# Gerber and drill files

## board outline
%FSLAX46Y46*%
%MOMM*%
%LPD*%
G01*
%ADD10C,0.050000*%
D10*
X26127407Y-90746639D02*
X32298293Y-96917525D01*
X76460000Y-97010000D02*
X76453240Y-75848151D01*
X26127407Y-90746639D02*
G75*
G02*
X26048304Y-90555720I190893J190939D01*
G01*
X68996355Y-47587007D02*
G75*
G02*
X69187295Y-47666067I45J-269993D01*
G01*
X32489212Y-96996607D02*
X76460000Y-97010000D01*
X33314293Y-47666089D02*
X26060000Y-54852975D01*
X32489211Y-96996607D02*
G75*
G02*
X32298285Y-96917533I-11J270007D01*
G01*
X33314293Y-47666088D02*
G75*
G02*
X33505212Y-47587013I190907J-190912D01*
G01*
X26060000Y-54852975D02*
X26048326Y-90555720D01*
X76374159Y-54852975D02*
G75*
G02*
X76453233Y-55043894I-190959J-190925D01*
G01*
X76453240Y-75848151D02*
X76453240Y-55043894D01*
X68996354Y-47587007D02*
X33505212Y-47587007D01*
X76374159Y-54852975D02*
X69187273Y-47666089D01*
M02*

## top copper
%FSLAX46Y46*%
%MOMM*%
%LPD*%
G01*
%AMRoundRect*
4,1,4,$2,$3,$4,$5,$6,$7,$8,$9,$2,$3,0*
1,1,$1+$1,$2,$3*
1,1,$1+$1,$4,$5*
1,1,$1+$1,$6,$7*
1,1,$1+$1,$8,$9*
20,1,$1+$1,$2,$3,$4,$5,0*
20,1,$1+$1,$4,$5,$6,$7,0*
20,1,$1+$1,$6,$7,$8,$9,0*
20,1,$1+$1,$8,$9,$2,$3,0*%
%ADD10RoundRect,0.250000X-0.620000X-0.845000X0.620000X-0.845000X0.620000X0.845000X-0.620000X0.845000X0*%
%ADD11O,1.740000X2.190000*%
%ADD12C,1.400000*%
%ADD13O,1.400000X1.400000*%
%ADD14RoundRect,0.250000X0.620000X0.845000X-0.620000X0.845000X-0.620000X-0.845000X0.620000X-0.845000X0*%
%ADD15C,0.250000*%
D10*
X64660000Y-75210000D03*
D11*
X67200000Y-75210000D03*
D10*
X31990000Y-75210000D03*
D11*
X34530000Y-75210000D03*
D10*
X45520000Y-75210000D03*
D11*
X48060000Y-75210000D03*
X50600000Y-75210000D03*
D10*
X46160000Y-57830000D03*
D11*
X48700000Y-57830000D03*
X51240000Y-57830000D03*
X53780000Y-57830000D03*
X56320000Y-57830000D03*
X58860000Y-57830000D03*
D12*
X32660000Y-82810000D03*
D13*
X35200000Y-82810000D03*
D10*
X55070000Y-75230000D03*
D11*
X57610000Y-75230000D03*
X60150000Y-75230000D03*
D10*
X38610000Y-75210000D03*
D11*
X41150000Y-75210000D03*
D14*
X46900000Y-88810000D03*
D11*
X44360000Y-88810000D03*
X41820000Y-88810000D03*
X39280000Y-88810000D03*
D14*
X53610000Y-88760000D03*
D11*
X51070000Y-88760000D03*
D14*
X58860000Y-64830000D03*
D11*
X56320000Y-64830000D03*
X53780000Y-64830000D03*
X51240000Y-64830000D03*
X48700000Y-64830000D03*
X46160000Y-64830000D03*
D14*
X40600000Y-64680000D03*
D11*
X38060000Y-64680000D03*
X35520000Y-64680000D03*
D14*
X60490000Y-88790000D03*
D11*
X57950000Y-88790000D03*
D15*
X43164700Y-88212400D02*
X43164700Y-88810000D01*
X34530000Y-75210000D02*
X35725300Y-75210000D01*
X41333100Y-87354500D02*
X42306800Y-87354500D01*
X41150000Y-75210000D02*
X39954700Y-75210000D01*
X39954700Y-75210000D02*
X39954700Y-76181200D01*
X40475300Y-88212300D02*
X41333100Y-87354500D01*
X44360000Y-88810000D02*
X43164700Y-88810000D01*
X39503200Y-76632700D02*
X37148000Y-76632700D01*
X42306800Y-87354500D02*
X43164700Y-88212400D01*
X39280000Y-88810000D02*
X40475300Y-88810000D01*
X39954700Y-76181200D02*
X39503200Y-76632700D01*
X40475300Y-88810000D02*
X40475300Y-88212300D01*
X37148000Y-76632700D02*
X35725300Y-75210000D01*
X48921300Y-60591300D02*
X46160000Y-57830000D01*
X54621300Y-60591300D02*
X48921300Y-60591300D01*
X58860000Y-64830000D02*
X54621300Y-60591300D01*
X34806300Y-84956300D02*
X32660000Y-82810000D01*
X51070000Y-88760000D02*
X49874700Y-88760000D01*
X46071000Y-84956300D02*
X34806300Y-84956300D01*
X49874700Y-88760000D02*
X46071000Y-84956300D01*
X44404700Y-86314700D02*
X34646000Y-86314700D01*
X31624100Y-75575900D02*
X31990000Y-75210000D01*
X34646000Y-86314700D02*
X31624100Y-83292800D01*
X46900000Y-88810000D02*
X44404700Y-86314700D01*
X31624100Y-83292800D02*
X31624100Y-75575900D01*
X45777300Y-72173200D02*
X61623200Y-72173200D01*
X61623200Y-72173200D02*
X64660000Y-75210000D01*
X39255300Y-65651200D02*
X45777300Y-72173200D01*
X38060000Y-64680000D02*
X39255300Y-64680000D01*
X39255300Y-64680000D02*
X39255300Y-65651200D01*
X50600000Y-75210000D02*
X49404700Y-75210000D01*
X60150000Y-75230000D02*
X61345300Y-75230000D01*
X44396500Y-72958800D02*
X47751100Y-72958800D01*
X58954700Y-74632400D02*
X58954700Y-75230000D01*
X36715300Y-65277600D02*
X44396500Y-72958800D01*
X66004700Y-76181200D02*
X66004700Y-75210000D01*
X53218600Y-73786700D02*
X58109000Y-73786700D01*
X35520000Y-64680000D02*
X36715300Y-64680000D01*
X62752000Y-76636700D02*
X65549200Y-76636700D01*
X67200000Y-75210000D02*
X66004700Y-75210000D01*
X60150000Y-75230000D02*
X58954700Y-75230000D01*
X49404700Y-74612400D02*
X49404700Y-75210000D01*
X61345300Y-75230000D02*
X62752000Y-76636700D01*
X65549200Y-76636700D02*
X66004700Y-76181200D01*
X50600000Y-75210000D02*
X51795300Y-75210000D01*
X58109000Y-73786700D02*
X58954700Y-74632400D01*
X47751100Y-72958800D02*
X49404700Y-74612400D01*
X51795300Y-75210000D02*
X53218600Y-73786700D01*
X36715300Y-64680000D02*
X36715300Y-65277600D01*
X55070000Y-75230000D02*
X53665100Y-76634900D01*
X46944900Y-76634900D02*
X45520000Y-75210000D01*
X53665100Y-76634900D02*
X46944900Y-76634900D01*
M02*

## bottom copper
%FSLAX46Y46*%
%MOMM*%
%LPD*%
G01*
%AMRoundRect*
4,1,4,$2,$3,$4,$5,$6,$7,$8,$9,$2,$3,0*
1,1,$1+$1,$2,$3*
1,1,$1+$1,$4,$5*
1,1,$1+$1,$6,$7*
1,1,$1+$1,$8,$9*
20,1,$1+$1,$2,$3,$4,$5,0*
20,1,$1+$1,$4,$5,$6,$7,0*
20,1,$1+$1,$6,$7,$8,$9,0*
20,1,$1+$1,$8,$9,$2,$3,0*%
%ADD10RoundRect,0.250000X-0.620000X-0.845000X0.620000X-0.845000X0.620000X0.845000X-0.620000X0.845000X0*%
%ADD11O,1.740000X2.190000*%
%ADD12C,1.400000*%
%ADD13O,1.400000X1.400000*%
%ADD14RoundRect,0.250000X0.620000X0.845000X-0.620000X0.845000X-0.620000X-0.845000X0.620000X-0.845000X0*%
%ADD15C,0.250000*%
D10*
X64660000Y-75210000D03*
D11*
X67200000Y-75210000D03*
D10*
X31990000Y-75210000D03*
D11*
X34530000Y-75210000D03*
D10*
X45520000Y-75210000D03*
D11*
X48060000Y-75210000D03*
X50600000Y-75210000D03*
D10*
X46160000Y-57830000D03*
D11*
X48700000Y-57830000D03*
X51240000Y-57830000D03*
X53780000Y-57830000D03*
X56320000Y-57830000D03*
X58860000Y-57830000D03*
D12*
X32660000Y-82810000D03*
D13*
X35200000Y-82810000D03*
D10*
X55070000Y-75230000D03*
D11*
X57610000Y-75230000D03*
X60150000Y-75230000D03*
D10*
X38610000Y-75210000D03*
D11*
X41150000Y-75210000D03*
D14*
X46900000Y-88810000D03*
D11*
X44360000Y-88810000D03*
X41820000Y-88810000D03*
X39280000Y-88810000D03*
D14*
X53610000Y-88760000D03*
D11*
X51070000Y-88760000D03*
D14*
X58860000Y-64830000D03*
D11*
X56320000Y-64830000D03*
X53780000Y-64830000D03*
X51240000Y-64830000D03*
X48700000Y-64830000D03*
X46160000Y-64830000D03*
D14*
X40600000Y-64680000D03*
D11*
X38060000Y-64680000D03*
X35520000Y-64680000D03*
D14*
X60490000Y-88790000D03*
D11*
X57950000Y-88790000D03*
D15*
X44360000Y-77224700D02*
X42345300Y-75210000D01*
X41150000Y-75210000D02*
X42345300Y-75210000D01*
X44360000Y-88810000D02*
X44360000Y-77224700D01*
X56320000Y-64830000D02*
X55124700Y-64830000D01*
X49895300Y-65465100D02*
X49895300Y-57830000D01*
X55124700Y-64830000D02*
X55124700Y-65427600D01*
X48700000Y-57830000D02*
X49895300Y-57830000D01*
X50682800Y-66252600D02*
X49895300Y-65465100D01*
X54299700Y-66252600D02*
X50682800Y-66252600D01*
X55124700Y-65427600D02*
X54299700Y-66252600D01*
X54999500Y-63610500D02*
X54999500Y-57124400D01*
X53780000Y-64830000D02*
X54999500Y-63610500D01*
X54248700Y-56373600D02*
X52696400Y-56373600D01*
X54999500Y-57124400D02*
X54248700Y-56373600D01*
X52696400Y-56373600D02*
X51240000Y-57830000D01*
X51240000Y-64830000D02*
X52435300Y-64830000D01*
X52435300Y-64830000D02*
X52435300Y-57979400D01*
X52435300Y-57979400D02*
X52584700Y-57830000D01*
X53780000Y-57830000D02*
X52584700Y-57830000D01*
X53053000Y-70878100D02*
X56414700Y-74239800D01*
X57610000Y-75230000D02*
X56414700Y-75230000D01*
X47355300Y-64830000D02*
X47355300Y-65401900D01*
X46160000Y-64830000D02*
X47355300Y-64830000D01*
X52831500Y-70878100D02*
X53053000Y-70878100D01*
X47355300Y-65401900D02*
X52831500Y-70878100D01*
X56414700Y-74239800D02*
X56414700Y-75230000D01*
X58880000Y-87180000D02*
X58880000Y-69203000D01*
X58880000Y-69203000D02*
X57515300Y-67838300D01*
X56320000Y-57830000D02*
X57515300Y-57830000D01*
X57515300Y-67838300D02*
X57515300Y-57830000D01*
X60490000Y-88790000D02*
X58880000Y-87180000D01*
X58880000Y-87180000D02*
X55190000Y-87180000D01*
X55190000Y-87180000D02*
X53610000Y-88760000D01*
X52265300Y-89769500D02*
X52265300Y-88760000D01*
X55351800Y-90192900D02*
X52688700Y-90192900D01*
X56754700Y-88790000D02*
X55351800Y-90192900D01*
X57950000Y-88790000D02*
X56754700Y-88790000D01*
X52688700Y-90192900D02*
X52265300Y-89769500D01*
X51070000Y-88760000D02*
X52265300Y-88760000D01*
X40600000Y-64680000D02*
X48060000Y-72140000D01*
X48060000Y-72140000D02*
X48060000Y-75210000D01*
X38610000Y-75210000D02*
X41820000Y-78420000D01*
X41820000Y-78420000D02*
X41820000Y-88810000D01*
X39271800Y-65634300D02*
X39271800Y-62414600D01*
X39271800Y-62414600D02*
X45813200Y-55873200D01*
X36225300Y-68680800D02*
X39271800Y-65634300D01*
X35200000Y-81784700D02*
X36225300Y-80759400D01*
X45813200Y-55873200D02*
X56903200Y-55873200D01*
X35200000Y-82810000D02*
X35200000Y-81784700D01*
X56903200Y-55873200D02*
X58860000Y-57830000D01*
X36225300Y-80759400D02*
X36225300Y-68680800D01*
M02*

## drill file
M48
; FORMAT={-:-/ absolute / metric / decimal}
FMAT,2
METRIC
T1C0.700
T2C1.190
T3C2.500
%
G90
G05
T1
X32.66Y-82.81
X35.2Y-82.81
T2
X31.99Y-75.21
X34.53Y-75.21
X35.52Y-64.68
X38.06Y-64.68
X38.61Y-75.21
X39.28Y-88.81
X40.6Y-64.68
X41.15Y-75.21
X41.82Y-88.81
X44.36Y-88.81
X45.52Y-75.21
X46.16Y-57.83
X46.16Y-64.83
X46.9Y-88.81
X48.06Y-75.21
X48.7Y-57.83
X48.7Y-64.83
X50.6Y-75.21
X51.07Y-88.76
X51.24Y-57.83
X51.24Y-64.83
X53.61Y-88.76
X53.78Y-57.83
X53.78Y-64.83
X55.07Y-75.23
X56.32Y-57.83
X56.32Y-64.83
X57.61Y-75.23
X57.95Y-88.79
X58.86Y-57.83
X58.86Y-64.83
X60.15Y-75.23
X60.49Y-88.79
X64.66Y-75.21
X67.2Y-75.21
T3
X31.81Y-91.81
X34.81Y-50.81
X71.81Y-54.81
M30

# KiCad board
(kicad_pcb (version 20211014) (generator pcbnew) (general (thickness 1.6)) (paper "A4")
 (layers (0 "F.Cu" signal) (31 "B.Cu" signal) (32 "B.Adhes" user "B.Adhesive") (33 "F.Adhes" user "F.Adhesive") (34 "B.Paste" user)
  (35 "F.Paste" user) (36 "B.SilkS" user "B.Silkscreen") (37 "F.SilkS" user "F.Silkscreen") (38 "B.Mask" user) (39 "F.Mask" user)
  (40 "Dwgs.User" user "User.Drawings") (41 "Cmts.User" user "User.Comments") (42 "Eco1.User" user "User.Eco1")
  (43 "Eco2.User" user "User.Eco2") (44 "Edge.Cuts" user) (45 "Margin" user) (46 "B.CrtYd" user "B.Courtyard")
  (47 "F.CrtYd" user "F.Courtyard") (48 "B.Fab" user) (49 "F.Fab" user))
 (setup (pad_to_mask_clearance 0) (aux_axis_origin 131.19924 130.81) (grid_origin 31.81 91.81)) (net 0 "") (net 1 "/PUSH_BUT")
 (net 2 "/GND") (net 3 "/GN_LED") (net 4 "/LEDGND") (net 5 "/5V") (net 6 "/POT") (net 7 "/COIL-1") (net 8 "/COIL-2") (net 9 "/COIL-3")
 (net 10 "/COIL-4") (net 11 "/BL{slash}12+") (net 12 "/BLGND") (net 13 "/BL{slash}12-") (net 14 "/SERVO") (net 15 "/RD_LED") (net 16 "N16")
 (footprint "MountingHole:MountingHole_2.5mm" (layer "F.Cu") (at 34.81 50.81)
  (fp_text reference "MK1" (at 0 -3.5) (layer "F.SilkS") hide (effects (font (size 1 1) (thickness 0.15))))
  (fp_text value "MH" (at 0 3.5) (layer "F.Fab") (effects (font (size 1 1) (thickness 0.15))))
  (pad "" np_thru_hole circle locked (at 0 0) (size 2.5 2.5) (drill 2.5) (layers *.Cu *.Mask)))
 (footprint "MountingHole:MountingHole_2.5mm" (layer "F.Cu") (at 31.81 91.81)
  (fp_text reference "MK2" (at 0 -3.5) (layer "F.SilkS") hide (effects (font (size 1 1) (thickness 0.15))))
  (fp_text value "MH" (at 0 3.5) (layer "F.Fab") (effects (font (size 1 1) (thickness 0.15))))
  (pad "" np_thru_hole circle locked (at 0 0) (size 2.5 2.5) (drill 2.5) (layers *.Cu *.Mask)))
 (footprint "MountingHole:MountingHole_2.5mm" (layer "F.Cu") (at 71.81 54.81)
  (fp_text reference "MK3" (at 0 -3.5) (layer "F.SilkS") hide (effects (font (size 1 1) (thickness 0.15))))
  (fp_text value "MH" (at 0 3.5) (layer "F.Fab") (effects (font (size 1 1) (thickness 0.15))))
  (pad "" np_thru_hole circle locked (at 0 0) (size 2.5 2.5) (drill 2.5) (layers *.Cu *.Mask)))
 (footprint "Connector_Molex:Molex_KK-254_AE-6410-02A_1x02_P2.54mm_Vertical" (layer "F.Cu") (at 64.66 75.21)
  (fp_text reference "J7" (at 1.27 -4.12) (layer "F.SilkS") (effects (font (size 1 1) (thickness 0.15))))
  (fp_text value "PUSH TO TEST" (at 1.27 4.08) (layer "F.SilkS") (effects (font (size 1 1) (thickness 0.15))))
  (pad "1" thru_hole roundrect (at 0 0) (size 1.74 2.19) (drill 1.19) (layers *.Cu *.Mask) (roundrect_rratio 0.1436781609)
   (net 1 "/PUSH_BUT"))
  (pad "2" thru_hole oval (at 2.54 0) (size 1.74 2.19) (drill 1.19) (layers *.Cu *.Mask) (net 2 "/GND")))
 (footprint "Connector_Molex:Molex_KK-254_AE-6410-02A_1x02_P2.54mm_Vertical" (layer "F.Cu") (at 31.99 75.21)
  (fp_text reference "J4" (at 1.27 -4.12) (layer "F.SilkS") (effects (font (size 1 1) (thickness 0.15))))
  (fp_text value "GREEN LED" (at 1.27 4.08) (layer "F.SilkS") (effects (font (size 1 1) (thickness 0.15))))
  (pad "1" thru_hole roundrect (at 0 0) (size 1.74 2.19) (drill 1.19) (layers *.Cu *.Mask) (roundrect_rratio 0.1436781609) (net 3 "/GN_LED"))
  (pad "2" thru_hole oval (at 2.54 0) (size 1.74 2.19) (drill 1.19) (layers *.Cu *.Mask) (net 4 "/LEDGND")))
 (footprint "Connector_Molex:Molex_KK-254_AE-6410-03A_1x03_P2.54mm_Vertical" (layer "F.Cu") (at 45.52 75.21)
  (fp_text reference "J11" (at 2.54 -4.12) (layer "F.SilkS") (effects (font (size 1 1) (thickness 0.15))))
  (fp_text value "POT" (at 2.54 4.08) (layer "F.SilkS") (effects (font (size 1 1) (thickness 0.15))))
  (pad "1" thru_hole roundrect (at 0 0) (size 1.74 2.19) (drill 1.19) (layers *.Cu *.Mask) (roundrect_rratio 0.1436781609) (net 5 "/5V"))
  (pad "2" thru_hole oval (at 2.54 0) (size 1.74 2.19) (drill 1.19) (layers *.Cu *.Mask) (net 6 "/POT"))
  (pad "3" thru_hole oval (at 5.08 0) (size 1.74 2.19) (drill 1.19) (layers *.Cu *.Mask) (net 2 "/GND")))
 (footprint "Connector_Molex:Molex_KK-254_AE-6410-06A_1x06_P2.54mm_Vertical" (layer "F.Cu") (at 46.16 57.83)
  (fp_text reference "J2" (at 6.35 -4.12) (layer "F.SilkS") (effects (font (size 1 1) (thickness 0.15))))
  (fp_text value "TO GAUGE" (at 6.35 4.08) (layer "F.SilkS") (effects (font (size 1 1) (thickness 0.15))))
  (pad "1" thru_hole roundrect (at 0 0) (size 1.74 2.19) (drill 1.19) (layers *.Cu *.Mask) (roundrect_rratio 0.1436781609) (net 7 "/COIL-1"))
  (pad "2" thru_hole oval (at 2.54 0) (size 1.74 2.19) (drill 1.19) (layers *.Cu *.Mask) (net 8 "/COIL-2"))
  (pad "3" thru_hole oval (at 5.08 0) (size 1.74 2.19) (drill 1.19) (layers *.Cu *.Mask) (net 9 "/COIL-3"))
  (pad "4" thru_hole oval (at 7.62 0) (size 1.74 2.19) (drill 1.19) (layers *.Cu *.Mask) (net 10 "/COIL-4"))
  (pad "5" thru_hole oval (at 10.16 0) (size 1.74 2.19) (drill 1.19) (layers *.Cu *.Mask) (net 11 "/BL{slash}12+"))
  (pad "6" thru_hole oval (at 12.7 0) (size 1.74 2.19) (drill 1.19) (layers *.Cu *.Mask) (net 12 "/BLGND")))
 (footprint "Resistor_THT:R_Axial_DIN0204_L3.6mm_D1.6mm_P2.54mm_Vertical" (layer "F.Cu") (at 32.66 82.81)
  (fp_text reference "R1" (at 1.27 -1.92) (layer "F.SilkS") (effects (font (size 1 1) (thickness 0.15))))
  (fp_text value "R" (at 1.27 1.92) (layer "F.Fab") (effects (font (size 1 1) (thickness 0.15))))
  (pad "1" thru_hole circle (at 0 0) (size 1.4 1.4) (drill 0.7) (layers *.Cu *.Mask) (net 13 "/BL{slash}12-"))
  (pad "2" thru_hole oval (at 2.54 0) (size 1.4 1.4) (drill 0.7) (layers *.Cu *.Mask) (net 12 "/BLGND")))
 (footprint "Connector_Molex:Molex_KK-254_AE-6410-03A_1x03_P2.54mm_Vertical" (layer "F.Cu") (at 55.07 75.23)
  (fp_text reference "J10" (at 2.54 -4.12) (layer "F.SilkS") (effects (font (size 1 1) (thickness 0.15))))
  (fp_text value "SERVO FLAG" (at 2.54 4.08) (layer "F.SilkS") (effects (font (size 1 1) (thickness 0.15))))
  (pad "1" thru_hole roundrect (at 0 0) (size 1.74 2.19) (drill 1.19) (layers *.Cu *.Mask) (roundrect_rratio 0.1436781609) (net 5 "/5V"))
  (pad "2" thru_hole oval (at 2.54 0) (size 1.74 2.19) (drill 1.19) (layers *.Cu *.Mask) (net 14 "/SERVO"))
  (pad "3" thru_hole oval (at 5.08 0) (size 1.74 2.19) (drill 1.19) (layers *.Cu *.Mask) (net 2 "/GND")))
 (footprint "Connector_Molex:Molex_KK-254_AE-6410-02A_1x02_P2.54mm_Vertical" (layer "F.Cu") (at 38.61 75.21)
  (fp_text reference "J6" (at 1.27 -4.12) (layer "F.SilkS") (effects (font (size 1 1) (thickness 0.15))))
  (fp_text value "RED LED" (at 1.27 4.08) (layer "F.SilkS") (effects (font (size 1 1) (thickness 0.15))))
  (pad "1" thru_hole roundrect (at 0 0) (size 1.74 2.19) (drill 1.19) (layers *.Cu *.Mask) (roundrect_rratio 0.1436781609)
   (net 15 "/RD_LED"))
  (pad "2" thru_hole oval (at 2.54 0) (size 1.74 2.19) (drill 1.19) (layers *.Cu *.Mask) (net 4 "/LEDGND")))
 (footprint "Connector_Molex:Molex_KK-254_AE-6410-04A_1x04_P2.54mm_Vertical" (layer "B.Cu") (at 46.9 88.81 180)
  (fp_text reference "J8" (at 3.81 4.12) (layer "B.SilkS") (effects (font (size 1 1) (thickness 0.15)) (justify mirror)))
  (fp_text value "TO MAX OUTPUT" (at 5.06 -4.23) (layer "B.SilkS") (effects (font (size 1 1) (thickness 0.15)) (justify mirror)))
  (pad "1" thru_hole roundrect (at 0 0 180) (size 1.74 2.19) (drill 1.19) (layers *.Cu *.Mask) (roundrect_rratio 0.1436781609)
   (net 3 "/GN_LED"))
  (pad "2" thru_hole oval (at 2.54 0 180) (size 1.74 2.19) (drill 1.19) (layers *.Cu *.Mask) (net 4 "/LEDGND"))
  (pad "3" thru_hole oval (at 5.08 0 180) (size 1.74 2.19) (drill 1.19) (layers *.Cu *.Mask) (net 15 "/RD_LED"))
  (pad "4" thru_hole oval (at 7.62 0 180) (size 1.74 2.19) (drill 1.19) (layers *.Cu *.Mask) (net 4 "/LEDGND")))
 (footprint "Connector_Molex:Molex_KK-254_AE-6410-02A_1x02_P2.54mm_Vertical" (layer "B.Cu") (at 53.61 88.76 180)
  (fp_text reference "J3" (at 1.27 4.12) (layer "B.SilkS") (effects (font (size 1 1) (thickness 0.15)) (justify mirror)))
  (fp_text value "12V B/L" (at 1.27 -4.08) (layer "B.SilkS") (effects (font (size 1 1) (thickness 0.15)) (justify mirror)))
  (pad "1" thru_hole roundrect (at 0 0 180) (size 1.74 2.19) (drill 1.19) (layers *.Cu *.Mask) (roundrect_rratio 0.1436781609)
   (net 11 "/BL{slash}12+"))
  (pad "2" thru_hole oval (at 2.54 0 180) (size 1.74 2.19) (drill 1.19) (layers *.Cu *.Mask) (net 13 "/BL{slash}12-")))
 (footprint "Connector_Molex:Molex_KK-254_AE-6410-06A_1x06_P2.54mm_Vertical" (layer "B.Cu") (at 58.86 64.83 180)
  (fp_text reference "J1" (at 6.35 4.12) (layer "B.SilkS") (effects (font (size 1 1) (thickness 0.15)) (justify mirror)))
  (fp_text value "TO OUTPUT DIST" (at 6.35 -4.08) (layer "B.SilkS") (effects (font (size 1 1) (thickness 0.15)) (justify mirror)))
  (pad "1" thru_hole roundrect (at 0 0 180) (size 1.74 2.19) (drill 1.19) (layers *.Cu *.Mask) (roundrect_rratio 0.1436781609)
   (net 7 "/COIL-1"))
  (pad "2" thru_hole oval (at 2.54 0 180) (size 1.74 2.19) (drill 1.19) (layers *.Cu *.Mask) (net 8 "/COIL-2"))
  (pad "3" thru_hole oval (at 5.08 0 180) (size 1.74 2.19) (drill 1.19) (layers *.Cu *.Mask) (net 9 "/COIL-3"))
  (pad "4" thru_hole oval (at 7.62 0 180) (size 1.74 2.19) (drill 1.19) (layers *.Cu *.Mask) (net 10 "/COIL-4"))
  (pad "5" thru_hole oval (at 10.16 0 180) (size 1.74 2.19) (drill 1.19) (layers *.Cu *.Mask) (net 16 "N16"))
  (pad "6" thru_hole oval (at 12.7 0 180) (size 1.74 2.19) (drill 1.19) (layers *.Cu *.Mask) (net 14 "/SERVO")))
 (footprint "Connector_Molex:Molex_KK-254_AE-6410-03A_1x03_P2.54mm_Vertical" (layer "B.Cu") (at 40.6 64.68 180)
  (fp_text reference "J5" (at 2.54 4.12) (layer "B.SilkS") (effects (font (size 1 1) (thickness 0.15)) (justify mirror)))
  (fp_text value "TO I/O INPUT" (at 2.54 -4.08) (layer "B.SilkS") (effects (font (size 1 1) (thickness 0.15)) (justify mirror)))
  (pad "1" thru_hole roundrect (at 0 0 180) (size 1.74 2.19) (drill 1.19) (layers *.Cu *.Mask) (roundrect_rratio 0.1436781609)
   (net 6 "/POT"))
  (pad "2" thru_hole oval (at 2.54 0 180) (size 1.74 2.19) (drill 1.19) (layers *.Cu *.Mask) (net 1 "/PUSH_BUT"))
  (pad "3" thru_hole oval (at 5.08 0 180) (size 1.74 2.19) (drill 1.19) (layers *.Cu *.Mask) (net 2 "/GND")))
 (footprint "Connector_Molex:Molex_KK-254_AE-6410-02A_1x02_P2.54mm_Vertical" (layer "B.Cu") (at 60.49 88.79 180)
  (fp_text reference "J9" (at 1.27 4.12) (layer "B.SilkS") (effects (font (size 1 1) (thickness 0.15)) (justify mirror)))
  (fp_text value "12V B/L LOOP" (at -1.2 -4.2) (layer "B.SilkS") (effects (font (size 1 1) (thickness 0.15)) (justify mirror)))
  (pad "1" thru_hole roundrect (at 0 0 180) (size 1.74 2.19) (drill 1.19) (layers *.Cu *.Mask) (roundrect_rratio 0.1436781609)
   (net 11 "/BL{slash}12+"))
  (pad "2" thru_hole oval (at 2.54 0 180) (size 1.74 2.19) (drill 1.19) (layers *.Cu *.Mask) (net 13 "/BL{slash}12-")))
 (gr_line (start 26.127407 90.746639) (end 32.298293 96.917525) (layer "Edge.Cuts") (width 0.05))
 (gr_line (start 76.46 97.01) (end 76.45324 75.848151) (layer "Edge.Cuts") (width 0.05))
 (gr_arc (start 26.127407 90.746639) (mid 26.068878 90.659045) (end 26.048326 90.55572) (layer "Edge.Cuts") (width 0.05))
 (gr_arc (start 68.996355 47.587007) (mid 69.099679 47.60756) (end 69.187273 47.666089) (layer "Edge.Cuts") (width 0.05))
 (gr_line (start 32.489212 96.996607) (end 76.46 97.01) (layer "Edge.Cuts") (width 0.05))
 (gr_line (start 33.314293 47.666089) (end 26.06 54.852975) (layer "Edge.Cuts") (width 0.05))
 (gr_arc (start 32.489211 96.996607) (mid 32.385887 96.976054) (end 32.298293 96.917525) (layer "Edge.Cuts") (width 0.05))
 (gr_arc (start 33.314293 47.666088) (mid 33.401887 47.607559) (end 33.505212 47.587007) (layer "Edge.Cuts") (width 0.05))
 (gr_line (start 26.06 54.852975) (end 26.048326 90.55572) (layer "Edge.Cuts") (width 0.05))
 (gr_arc (start 76.374159 54.852975) (mid 76.432688 54.940569) (end 76.45324 55.043894) (layer "Edge.Cuts") (width 0.05))
 (gr_line (start 76.45324 75.848151) (end 76.45324 55.043894) (layer "Edge.Cuts") (width 0.05))
 (gr_line (start 68.996354 47.587007) (end 33.505212 47.587007) (layer "Edge.Cuts") (width 0.05))
 (gr_line (start 76.374159 54.852975) (end 69.187273 47.666089) (layer "Edge.Cuts") (width 0.05))
 (segment (start 43.1647 88.2124) (end 43.1647 88.81) (width 0.25) (layer "F.Cu") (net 4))
 (segment (start 34.53 75.21) (end 35.7253 75.21) (width 0.25) (layer "F.Cu") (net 4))
 (segment (start 41.3331 87.3545) (end 42.3068 87.3545) (width 0.25) (layer "F.Cu") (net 4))
 (segment (start 41.15 75.21) (end 39.9547 75.21) (width 0.25) (layer "F.Cu") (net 4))
 (segment (start 39.9547 75.21) (end 39.9547 76.1812) (width 0.25) (layer "F.Cu") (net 4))
 (segment (start 40.4753 88.2123) (end 41.3331 87.3545) (width 0.25) (layer "F.Cu") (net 4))
 (segment (start 44.36 88.81) (end 43.1647 88.81) (width 0.25) (layer "F.Cu") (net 4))
 (segment (start 39.5032 76.6327) (end 37.148 76.6327) (width 0.25) (layer "F.Cu") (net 4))
 (segment (start 42.3068 87.3545) (end 43.1647 88.2124) (width 0.25) (layer "F.Cu") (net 4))
 (segment (start 39.28 88.81) (end 40.4753 88.81) (width 0.25) (layer "F.Cu") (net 4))
 (segment (start 39.9547 76.1812) (end 39.5032 76.6327) (width 0.25) (layer "F.Cu") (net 4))
 (segment (start 40.4753 88.81) (end 40.4753 88.2123) (width 0.25) (layer "F.Cu") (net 4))
 (segment (start 37.148 76.6327) (end 35.7253 75.21) (width 0.25) (layer "F.Cu") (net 4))
 (segment (start 44.36 77.2247) (end 42.3453 75.21) (width 0.25) (layer "B.Cu") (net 4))
 (segment (start 41.15 75.21) (end 42.3453 75.21) (width 0.25) (layer "B.Cu") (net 4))
 (segment (start 44.36 88.81) (end 44.36 77.2247) (width 0.25) (layer "B.Cu") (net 4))
 (segment (start 48.9213 60.5913) (end 46.16 57.83) (width 0.25) (layer "F.Cu") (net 7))
 (segment (start 54.6213 60.5913) (end 48.9213 60.5913) (width 0.25) (layer "F.Cu") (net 7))
 (segment (start 58.86 64.83) (end 54.6213 60.5913) (width 0.25) (layer "F.Cu") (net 7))
 (segment (start 56.32 64.83) (end 55.1247 64.83) (width 0.25) (layer "B.Cu") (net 8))
 (segment (start 49.8953 65.4651) (end 49.8953 57.83) (width 0.25) (layer "B.Cu") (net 8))
 (segment (start 55.1247 64.83) (end 55.1247 65.4276) (width 0.25) (layer "B.Cu") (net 8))
 (segment (start 48.7 57.83) (end 49.8953 57.83) (width 0.25) (layer "B.Cu") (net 8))
 (segment (start 50.6828 66.2526) (end 49.8953 65.4651) (width 0.25) (layer "B.Cu") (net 8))
 (segment (start 54.2997 66.2526) (end 50.6828 66.2526) (width 0.25) (layer "B.Cu") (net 8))
 (segment (start 55.1247 65.4276) (end 54.2997 66.2526) (width 0.25) (layer "B.Cu") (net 8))
 (segment (start 54.9995 63.6105) (end 54.9995 57.1244) (width 0.25) (layer "B.Cu") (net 9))
 (segment (start 53.78 64.83) (end 54.9995 63.6105) (width 0.25) (layer "B.Cu") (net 9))
 (segment (start 54.2487 56.3736) (end 52.6964 56.3736) (width 0.25) (layer "B.Cu") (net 9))
 (segment (start 54.9995 57.1244) (end 54.2487 56.3736) (width 0.25) (layer "B.Cu") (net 9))
 (segment (start 52.6964 56.3736) (end 51.24 57.83) (width 0.25) (layer "B.Cu") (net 9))
 (segment (start 51.24 64.83) (end 52.4353 64.83) (width 0.25) (layer "B.Cu") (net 10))
 (segment (start 52.4353 64.83) (end 52.4353 57.9794) (width 0.25) (layer "B.Cu") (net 10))
 (segment (start 52.4353 57.9794) (end 52.5847 57.83) (width 0.25) (layer "B.Cu") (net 10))
 (segment (start 53.78 57.83) (end 52.5847 57.83) (width 0.25) (layer "B.Cu") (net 10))
 (segment (start 53.053 70.8781) (end 56.4147 74.2398) (width 0.25) (layer "B.Cu") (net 14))
 (segment (start 57.61 75.23) (end 56.4147 75.23) (width 0.25) (layer "B.Cu") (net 14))
 (segment (start 47.3553 64.83) (end 47.3553 65.4019) (width 0.25) (layer "B.Cu") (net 14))
 (segment (start 46.16 64.83) (end 47.3553 64.83) (width 0.25) (layer "B.Cu") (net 14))
 (segment (start 52.8315 70.8781) (end 53.053 70.8781) (width 0.25) (layer "B.Cu") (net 14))
 (segment (start 47.3553 65.4019) (end 52.8315 70.8781) (width 0.25) (layer "B.Cu") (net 14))
 (segment (start 56.4147 74.2398) (end 56.4147 75.23) (width 0.25) (layer "B.Cu") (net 14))
 (segment (start 58.88 87.18) (end 58.88 69.203) (width 0.25) (layer "B.Cu") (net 11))
 (segment (start 58.88 69.203) (end 57.5153 67.8383) (width 0.25) (layer "B.Cu") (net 11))
 (segment (start 56.32 57.83) (end 57.5153 57.83) (width 0.25) (layer "B.Cu") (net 11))
 (segment (start 57.5153 67.8383) (end 57.5153 57.83) (width 0.25) (layer "B.Cu") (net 11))
 (segment (start 60.49 88.79) (end 58.88 87.18) (width 0.25) (layer "B.Cu") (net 11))
 (segment (start 58.88 87.18) (end 55.19 87.18) (width 0.25) (layer "B.Cu") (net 11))
 (segment (start 55.19 87.18) (end 53.61 88.76) (width 0.25) (layer "B.Cu") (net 11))
 (segment (start 34.8063 84.9563) (end 32.66 82.81) (width 0.25) (layer "F.Cu") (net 13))
 (segment (start 51.07 88.76) (end 49.8747 88.76) (width 0.25) (layer "F.Cu") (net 13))
 (segment (start 46.071 84.9563) (end 34.8063 84.9563) (width 0.25) (layer "F.Cu") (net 13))
 (segment (start 49.8747 88.76) (end 46.071 84.9563) (width 0.25) (layer "F.Cu") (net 13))
 (segment (start 52.2653 89.7695) (end 52.2653 88.76) (width 0.25) (layer "B.Cu") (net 13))
 (segment (start 55.3518 90.1929) (end 52.6887 90.1929) (width 0.25) (layer "B.Cu") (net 13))
 (segment (start 56.7547 88.79) (end 55.3518 90.1929) (width 0.25) (layer "B.Cu") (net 13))
 (segment (start 57.95 88.79) (end 56.7547 88.79) (width 0.25) (layer "B.Cu") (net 13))
 (segment (start 52.6887 90.1929) (end 52.2653 89.7695) (width 0.25) (layer "B.Cu") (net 13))
 (segment (start 51.07 88.76) (end 52.2653 88.76) (width 0.25) (layer "B.Cu") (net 13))
 (segment (start 44.4047 86.3147) (end 34.646 86.3147) (width 0.25) (layer "F.Cu") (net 3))
 (segment (start 31.6241 75.5759) (end 31.99 75.21) (width 0.25) (layer "F.Cu") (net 3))
 (segment (start 34.646 86.3147) (end 31.6241 83.2928) (width 0.25) (layer "F.Cu") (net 3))
 (segment (start 46.9 88.81) (end 44.4047 86.3147) (width 0.25) (layer "F.Cu") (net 3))
 (segment (start 31.6241 83.2928) (end 31.6241 75.5759) (width 0.25) (layer "F.Cu") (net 3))
 (segment (start 40.6 64.68) (end 48.06 72.14) (width 0.25) (layer "B.Cu") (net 6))
 (segment (start 48.06 72.14) (end 48.06 75.21) (width 0.25) (layer "B.Cu") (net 6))
 (segment (start 45.7773 72.1732) (end 61.6232 72.1732) (width 0.25) (layer "F.Cu") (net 1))
 (segment (start 61.6232 72.1732) (end 64.66 75.21) (width 0.25) (layer "F.Cu") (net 1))
 (segment (start 39.2553 65.6512) (end 45.7773 72.1732) (width 0.25) (layer "F.Cu") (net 1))
 (segment (start 38.06 64.68) (end 39.2553 64.68) (width 0.25) (layer "F.Cu") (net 1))
 (segment (start 39.2553 64.68) (end 39.2553 65.6512) (width 0.25) (layer "F.Cu") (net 1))
 (segment (start 50.6 75.21) (end 49.4047 75.21) (width 0.25) (layer "F.Cu") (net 2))
 (segment (start 60.15 75.23) (end 61.3453 75.23) (width 0.25) (layer "F.Cu") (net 2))
 (segment (start 44.3965 72.9588) (end 47.7511 72.9588) (width 0.25) (layer "F.Cu") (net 2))
 (segment (start 58.9547 74.6324) (end 58.9547 75.23) (width 0.25) (layer "F.Cu") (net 2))
 (segment (start 36.7153 65.2776) (end 44.3965 72.9588) (width 0.25) (layer "F.Cu") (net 2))
 (segment (start 66.0047 76.1812) (end 66.0047 75.21) (width 0.25) (layer "F.Cu") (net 2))
 (segment (start 53.2186 73.7867) (end 58.109 73.7867) (width 0.25) (layer "F.Cu") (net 2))
 (segment (start 35.52 64.68) (end 36.7153 64.68) (width 0.25) (layer "F.Cu") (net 2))
 (segment (start 62.752 76.6367) (end 65.5492 76.6367) (width 0.25) (layer "F.Cu") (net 2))
 (segment (start 67.2 75.21) (end 66.0047 75.21) (width 0.25) (layer "F.Cu") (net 2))
 (segment (start 60.15 75.23) (end 58.9547 75.23) (width 0.25) (layer "F.Cu") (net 2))
 (segment (start 49.4047 74.6124) (end 49.4047 75.21) (width 0.25) (layer "F.Cu") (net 2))
 (segment (start 61.3453 75.23) (end 62.752 76.6367) (width 0.25) (layer "F.Cu") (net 2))
 (segment (start 65.5492 76.6367) (end 66.0047 76.1812) (width 0.25) (layer "F.Cu") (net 2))
 (segment (start 50.6 75.21) (end 51.7953 75.21) (width 0.25) (layer "F.Cu") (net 2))
 (segment (start 58.109 73.7867) (end 58.9547 74.6324) (width 0.25) (layer "F.Cu") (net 2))
 (segment (start 47.7511 72.9588) (end 49.4047 74.6124) (width 0.25) (layer "F.Cu") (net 2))
 (segment (start 51.7953 75.21) (end 53.2186 73.7867) (width 0.25) (layer "F.Cu") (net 2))
 (segment (start 36.7153 64.68) (end 36.7153 65.2776) (width 0.25) (layer "F.Cu") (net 2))
 (segment (start 38.61 75.21) (end 41.82 78.42) (width 0.25) (layer "B.Cu") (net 15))
 (segment (start 41.82 78.42) (end 41.82 88.81) (width 0.25) (layer "B.Cu") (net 15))
 (segment (start 55.07 75.23) (end 53.6651 76.6349) (width 0.25) (layer "F.Cu") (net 5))
 (segment (start 46.9449 76.6349) (end 45.52 75.21) (width 0.25) (layer "F.Cu") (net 5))
 (segment (start 53.6651 76.6349) (end 46.9449 76.6349) (width 0.25) (layer "F.Cu") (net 5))
 (segment (start 39.2718 65.6343) (end 39.2718 62.4146) (width 0.25) (layer "B.Cu") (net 12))
 (segment (start 39.2718 62.4146) (end 45.8132 55.8732) (width 0.25) (layer "B.Cu") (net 12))
 (segment (start 36.2253 68.6808) (end 39.2718 65.6343) (width 0.25) (layer "B.Cu") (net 12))
 (segment (start 35.2 81.7847) (end 36.2253 80.7594) (width 0.25) (layer "B.Cu") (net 12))
 (segment (start 45.8132 55.8732) (end 56.9032 55.8732) (width 0.25) (layer "B.Cu") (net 12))
 (segment (start 35.2 82.81) (end 35.2 81.7847) (width 0.25) (layer "B.Cu") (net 12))
 (segment (start 56.9032 55.8732) (end 58.86 57.83) (width 0.25) (layer "B.Cu") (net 12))
 (segment (start 36.2253 80.7594) (end 36.2253 68.6808) (width 0.25) (layer "B.Cu") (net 12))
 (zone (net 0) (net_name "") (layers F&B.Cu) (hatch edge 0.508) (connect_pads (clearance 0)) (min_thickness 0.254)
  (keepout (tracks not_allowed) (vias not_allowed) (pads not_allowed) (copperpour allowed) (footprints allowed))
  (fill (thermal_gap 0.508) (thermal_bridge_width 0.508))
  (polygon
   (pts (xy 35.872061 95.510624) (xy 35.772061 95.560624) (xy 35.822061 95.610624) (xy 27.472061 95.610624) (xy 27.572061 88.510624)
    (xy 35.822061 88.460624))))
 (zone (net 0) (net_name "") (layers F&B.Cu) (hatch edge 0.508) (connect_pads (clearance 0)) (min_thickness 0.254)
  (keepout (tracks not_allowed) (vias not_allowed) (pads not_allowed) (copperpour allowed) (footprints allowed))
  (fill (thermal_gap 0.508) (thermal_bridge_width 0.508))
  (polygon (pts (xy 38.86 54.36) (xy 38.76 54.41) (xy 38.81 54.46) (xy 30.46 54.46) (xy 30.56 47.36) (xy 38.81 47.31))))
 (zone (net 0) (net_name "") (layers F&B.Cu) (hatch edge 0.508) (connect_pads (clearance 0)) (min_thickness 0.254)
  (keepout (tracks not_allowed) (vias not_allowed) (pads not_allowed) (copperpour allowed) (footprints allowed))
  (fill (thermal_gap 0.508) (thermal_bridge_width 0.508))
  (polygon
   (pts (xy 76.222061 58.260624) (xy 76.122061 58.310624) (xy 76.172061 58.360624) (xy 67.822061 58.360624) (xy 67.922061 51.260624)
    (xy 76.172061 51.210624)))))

